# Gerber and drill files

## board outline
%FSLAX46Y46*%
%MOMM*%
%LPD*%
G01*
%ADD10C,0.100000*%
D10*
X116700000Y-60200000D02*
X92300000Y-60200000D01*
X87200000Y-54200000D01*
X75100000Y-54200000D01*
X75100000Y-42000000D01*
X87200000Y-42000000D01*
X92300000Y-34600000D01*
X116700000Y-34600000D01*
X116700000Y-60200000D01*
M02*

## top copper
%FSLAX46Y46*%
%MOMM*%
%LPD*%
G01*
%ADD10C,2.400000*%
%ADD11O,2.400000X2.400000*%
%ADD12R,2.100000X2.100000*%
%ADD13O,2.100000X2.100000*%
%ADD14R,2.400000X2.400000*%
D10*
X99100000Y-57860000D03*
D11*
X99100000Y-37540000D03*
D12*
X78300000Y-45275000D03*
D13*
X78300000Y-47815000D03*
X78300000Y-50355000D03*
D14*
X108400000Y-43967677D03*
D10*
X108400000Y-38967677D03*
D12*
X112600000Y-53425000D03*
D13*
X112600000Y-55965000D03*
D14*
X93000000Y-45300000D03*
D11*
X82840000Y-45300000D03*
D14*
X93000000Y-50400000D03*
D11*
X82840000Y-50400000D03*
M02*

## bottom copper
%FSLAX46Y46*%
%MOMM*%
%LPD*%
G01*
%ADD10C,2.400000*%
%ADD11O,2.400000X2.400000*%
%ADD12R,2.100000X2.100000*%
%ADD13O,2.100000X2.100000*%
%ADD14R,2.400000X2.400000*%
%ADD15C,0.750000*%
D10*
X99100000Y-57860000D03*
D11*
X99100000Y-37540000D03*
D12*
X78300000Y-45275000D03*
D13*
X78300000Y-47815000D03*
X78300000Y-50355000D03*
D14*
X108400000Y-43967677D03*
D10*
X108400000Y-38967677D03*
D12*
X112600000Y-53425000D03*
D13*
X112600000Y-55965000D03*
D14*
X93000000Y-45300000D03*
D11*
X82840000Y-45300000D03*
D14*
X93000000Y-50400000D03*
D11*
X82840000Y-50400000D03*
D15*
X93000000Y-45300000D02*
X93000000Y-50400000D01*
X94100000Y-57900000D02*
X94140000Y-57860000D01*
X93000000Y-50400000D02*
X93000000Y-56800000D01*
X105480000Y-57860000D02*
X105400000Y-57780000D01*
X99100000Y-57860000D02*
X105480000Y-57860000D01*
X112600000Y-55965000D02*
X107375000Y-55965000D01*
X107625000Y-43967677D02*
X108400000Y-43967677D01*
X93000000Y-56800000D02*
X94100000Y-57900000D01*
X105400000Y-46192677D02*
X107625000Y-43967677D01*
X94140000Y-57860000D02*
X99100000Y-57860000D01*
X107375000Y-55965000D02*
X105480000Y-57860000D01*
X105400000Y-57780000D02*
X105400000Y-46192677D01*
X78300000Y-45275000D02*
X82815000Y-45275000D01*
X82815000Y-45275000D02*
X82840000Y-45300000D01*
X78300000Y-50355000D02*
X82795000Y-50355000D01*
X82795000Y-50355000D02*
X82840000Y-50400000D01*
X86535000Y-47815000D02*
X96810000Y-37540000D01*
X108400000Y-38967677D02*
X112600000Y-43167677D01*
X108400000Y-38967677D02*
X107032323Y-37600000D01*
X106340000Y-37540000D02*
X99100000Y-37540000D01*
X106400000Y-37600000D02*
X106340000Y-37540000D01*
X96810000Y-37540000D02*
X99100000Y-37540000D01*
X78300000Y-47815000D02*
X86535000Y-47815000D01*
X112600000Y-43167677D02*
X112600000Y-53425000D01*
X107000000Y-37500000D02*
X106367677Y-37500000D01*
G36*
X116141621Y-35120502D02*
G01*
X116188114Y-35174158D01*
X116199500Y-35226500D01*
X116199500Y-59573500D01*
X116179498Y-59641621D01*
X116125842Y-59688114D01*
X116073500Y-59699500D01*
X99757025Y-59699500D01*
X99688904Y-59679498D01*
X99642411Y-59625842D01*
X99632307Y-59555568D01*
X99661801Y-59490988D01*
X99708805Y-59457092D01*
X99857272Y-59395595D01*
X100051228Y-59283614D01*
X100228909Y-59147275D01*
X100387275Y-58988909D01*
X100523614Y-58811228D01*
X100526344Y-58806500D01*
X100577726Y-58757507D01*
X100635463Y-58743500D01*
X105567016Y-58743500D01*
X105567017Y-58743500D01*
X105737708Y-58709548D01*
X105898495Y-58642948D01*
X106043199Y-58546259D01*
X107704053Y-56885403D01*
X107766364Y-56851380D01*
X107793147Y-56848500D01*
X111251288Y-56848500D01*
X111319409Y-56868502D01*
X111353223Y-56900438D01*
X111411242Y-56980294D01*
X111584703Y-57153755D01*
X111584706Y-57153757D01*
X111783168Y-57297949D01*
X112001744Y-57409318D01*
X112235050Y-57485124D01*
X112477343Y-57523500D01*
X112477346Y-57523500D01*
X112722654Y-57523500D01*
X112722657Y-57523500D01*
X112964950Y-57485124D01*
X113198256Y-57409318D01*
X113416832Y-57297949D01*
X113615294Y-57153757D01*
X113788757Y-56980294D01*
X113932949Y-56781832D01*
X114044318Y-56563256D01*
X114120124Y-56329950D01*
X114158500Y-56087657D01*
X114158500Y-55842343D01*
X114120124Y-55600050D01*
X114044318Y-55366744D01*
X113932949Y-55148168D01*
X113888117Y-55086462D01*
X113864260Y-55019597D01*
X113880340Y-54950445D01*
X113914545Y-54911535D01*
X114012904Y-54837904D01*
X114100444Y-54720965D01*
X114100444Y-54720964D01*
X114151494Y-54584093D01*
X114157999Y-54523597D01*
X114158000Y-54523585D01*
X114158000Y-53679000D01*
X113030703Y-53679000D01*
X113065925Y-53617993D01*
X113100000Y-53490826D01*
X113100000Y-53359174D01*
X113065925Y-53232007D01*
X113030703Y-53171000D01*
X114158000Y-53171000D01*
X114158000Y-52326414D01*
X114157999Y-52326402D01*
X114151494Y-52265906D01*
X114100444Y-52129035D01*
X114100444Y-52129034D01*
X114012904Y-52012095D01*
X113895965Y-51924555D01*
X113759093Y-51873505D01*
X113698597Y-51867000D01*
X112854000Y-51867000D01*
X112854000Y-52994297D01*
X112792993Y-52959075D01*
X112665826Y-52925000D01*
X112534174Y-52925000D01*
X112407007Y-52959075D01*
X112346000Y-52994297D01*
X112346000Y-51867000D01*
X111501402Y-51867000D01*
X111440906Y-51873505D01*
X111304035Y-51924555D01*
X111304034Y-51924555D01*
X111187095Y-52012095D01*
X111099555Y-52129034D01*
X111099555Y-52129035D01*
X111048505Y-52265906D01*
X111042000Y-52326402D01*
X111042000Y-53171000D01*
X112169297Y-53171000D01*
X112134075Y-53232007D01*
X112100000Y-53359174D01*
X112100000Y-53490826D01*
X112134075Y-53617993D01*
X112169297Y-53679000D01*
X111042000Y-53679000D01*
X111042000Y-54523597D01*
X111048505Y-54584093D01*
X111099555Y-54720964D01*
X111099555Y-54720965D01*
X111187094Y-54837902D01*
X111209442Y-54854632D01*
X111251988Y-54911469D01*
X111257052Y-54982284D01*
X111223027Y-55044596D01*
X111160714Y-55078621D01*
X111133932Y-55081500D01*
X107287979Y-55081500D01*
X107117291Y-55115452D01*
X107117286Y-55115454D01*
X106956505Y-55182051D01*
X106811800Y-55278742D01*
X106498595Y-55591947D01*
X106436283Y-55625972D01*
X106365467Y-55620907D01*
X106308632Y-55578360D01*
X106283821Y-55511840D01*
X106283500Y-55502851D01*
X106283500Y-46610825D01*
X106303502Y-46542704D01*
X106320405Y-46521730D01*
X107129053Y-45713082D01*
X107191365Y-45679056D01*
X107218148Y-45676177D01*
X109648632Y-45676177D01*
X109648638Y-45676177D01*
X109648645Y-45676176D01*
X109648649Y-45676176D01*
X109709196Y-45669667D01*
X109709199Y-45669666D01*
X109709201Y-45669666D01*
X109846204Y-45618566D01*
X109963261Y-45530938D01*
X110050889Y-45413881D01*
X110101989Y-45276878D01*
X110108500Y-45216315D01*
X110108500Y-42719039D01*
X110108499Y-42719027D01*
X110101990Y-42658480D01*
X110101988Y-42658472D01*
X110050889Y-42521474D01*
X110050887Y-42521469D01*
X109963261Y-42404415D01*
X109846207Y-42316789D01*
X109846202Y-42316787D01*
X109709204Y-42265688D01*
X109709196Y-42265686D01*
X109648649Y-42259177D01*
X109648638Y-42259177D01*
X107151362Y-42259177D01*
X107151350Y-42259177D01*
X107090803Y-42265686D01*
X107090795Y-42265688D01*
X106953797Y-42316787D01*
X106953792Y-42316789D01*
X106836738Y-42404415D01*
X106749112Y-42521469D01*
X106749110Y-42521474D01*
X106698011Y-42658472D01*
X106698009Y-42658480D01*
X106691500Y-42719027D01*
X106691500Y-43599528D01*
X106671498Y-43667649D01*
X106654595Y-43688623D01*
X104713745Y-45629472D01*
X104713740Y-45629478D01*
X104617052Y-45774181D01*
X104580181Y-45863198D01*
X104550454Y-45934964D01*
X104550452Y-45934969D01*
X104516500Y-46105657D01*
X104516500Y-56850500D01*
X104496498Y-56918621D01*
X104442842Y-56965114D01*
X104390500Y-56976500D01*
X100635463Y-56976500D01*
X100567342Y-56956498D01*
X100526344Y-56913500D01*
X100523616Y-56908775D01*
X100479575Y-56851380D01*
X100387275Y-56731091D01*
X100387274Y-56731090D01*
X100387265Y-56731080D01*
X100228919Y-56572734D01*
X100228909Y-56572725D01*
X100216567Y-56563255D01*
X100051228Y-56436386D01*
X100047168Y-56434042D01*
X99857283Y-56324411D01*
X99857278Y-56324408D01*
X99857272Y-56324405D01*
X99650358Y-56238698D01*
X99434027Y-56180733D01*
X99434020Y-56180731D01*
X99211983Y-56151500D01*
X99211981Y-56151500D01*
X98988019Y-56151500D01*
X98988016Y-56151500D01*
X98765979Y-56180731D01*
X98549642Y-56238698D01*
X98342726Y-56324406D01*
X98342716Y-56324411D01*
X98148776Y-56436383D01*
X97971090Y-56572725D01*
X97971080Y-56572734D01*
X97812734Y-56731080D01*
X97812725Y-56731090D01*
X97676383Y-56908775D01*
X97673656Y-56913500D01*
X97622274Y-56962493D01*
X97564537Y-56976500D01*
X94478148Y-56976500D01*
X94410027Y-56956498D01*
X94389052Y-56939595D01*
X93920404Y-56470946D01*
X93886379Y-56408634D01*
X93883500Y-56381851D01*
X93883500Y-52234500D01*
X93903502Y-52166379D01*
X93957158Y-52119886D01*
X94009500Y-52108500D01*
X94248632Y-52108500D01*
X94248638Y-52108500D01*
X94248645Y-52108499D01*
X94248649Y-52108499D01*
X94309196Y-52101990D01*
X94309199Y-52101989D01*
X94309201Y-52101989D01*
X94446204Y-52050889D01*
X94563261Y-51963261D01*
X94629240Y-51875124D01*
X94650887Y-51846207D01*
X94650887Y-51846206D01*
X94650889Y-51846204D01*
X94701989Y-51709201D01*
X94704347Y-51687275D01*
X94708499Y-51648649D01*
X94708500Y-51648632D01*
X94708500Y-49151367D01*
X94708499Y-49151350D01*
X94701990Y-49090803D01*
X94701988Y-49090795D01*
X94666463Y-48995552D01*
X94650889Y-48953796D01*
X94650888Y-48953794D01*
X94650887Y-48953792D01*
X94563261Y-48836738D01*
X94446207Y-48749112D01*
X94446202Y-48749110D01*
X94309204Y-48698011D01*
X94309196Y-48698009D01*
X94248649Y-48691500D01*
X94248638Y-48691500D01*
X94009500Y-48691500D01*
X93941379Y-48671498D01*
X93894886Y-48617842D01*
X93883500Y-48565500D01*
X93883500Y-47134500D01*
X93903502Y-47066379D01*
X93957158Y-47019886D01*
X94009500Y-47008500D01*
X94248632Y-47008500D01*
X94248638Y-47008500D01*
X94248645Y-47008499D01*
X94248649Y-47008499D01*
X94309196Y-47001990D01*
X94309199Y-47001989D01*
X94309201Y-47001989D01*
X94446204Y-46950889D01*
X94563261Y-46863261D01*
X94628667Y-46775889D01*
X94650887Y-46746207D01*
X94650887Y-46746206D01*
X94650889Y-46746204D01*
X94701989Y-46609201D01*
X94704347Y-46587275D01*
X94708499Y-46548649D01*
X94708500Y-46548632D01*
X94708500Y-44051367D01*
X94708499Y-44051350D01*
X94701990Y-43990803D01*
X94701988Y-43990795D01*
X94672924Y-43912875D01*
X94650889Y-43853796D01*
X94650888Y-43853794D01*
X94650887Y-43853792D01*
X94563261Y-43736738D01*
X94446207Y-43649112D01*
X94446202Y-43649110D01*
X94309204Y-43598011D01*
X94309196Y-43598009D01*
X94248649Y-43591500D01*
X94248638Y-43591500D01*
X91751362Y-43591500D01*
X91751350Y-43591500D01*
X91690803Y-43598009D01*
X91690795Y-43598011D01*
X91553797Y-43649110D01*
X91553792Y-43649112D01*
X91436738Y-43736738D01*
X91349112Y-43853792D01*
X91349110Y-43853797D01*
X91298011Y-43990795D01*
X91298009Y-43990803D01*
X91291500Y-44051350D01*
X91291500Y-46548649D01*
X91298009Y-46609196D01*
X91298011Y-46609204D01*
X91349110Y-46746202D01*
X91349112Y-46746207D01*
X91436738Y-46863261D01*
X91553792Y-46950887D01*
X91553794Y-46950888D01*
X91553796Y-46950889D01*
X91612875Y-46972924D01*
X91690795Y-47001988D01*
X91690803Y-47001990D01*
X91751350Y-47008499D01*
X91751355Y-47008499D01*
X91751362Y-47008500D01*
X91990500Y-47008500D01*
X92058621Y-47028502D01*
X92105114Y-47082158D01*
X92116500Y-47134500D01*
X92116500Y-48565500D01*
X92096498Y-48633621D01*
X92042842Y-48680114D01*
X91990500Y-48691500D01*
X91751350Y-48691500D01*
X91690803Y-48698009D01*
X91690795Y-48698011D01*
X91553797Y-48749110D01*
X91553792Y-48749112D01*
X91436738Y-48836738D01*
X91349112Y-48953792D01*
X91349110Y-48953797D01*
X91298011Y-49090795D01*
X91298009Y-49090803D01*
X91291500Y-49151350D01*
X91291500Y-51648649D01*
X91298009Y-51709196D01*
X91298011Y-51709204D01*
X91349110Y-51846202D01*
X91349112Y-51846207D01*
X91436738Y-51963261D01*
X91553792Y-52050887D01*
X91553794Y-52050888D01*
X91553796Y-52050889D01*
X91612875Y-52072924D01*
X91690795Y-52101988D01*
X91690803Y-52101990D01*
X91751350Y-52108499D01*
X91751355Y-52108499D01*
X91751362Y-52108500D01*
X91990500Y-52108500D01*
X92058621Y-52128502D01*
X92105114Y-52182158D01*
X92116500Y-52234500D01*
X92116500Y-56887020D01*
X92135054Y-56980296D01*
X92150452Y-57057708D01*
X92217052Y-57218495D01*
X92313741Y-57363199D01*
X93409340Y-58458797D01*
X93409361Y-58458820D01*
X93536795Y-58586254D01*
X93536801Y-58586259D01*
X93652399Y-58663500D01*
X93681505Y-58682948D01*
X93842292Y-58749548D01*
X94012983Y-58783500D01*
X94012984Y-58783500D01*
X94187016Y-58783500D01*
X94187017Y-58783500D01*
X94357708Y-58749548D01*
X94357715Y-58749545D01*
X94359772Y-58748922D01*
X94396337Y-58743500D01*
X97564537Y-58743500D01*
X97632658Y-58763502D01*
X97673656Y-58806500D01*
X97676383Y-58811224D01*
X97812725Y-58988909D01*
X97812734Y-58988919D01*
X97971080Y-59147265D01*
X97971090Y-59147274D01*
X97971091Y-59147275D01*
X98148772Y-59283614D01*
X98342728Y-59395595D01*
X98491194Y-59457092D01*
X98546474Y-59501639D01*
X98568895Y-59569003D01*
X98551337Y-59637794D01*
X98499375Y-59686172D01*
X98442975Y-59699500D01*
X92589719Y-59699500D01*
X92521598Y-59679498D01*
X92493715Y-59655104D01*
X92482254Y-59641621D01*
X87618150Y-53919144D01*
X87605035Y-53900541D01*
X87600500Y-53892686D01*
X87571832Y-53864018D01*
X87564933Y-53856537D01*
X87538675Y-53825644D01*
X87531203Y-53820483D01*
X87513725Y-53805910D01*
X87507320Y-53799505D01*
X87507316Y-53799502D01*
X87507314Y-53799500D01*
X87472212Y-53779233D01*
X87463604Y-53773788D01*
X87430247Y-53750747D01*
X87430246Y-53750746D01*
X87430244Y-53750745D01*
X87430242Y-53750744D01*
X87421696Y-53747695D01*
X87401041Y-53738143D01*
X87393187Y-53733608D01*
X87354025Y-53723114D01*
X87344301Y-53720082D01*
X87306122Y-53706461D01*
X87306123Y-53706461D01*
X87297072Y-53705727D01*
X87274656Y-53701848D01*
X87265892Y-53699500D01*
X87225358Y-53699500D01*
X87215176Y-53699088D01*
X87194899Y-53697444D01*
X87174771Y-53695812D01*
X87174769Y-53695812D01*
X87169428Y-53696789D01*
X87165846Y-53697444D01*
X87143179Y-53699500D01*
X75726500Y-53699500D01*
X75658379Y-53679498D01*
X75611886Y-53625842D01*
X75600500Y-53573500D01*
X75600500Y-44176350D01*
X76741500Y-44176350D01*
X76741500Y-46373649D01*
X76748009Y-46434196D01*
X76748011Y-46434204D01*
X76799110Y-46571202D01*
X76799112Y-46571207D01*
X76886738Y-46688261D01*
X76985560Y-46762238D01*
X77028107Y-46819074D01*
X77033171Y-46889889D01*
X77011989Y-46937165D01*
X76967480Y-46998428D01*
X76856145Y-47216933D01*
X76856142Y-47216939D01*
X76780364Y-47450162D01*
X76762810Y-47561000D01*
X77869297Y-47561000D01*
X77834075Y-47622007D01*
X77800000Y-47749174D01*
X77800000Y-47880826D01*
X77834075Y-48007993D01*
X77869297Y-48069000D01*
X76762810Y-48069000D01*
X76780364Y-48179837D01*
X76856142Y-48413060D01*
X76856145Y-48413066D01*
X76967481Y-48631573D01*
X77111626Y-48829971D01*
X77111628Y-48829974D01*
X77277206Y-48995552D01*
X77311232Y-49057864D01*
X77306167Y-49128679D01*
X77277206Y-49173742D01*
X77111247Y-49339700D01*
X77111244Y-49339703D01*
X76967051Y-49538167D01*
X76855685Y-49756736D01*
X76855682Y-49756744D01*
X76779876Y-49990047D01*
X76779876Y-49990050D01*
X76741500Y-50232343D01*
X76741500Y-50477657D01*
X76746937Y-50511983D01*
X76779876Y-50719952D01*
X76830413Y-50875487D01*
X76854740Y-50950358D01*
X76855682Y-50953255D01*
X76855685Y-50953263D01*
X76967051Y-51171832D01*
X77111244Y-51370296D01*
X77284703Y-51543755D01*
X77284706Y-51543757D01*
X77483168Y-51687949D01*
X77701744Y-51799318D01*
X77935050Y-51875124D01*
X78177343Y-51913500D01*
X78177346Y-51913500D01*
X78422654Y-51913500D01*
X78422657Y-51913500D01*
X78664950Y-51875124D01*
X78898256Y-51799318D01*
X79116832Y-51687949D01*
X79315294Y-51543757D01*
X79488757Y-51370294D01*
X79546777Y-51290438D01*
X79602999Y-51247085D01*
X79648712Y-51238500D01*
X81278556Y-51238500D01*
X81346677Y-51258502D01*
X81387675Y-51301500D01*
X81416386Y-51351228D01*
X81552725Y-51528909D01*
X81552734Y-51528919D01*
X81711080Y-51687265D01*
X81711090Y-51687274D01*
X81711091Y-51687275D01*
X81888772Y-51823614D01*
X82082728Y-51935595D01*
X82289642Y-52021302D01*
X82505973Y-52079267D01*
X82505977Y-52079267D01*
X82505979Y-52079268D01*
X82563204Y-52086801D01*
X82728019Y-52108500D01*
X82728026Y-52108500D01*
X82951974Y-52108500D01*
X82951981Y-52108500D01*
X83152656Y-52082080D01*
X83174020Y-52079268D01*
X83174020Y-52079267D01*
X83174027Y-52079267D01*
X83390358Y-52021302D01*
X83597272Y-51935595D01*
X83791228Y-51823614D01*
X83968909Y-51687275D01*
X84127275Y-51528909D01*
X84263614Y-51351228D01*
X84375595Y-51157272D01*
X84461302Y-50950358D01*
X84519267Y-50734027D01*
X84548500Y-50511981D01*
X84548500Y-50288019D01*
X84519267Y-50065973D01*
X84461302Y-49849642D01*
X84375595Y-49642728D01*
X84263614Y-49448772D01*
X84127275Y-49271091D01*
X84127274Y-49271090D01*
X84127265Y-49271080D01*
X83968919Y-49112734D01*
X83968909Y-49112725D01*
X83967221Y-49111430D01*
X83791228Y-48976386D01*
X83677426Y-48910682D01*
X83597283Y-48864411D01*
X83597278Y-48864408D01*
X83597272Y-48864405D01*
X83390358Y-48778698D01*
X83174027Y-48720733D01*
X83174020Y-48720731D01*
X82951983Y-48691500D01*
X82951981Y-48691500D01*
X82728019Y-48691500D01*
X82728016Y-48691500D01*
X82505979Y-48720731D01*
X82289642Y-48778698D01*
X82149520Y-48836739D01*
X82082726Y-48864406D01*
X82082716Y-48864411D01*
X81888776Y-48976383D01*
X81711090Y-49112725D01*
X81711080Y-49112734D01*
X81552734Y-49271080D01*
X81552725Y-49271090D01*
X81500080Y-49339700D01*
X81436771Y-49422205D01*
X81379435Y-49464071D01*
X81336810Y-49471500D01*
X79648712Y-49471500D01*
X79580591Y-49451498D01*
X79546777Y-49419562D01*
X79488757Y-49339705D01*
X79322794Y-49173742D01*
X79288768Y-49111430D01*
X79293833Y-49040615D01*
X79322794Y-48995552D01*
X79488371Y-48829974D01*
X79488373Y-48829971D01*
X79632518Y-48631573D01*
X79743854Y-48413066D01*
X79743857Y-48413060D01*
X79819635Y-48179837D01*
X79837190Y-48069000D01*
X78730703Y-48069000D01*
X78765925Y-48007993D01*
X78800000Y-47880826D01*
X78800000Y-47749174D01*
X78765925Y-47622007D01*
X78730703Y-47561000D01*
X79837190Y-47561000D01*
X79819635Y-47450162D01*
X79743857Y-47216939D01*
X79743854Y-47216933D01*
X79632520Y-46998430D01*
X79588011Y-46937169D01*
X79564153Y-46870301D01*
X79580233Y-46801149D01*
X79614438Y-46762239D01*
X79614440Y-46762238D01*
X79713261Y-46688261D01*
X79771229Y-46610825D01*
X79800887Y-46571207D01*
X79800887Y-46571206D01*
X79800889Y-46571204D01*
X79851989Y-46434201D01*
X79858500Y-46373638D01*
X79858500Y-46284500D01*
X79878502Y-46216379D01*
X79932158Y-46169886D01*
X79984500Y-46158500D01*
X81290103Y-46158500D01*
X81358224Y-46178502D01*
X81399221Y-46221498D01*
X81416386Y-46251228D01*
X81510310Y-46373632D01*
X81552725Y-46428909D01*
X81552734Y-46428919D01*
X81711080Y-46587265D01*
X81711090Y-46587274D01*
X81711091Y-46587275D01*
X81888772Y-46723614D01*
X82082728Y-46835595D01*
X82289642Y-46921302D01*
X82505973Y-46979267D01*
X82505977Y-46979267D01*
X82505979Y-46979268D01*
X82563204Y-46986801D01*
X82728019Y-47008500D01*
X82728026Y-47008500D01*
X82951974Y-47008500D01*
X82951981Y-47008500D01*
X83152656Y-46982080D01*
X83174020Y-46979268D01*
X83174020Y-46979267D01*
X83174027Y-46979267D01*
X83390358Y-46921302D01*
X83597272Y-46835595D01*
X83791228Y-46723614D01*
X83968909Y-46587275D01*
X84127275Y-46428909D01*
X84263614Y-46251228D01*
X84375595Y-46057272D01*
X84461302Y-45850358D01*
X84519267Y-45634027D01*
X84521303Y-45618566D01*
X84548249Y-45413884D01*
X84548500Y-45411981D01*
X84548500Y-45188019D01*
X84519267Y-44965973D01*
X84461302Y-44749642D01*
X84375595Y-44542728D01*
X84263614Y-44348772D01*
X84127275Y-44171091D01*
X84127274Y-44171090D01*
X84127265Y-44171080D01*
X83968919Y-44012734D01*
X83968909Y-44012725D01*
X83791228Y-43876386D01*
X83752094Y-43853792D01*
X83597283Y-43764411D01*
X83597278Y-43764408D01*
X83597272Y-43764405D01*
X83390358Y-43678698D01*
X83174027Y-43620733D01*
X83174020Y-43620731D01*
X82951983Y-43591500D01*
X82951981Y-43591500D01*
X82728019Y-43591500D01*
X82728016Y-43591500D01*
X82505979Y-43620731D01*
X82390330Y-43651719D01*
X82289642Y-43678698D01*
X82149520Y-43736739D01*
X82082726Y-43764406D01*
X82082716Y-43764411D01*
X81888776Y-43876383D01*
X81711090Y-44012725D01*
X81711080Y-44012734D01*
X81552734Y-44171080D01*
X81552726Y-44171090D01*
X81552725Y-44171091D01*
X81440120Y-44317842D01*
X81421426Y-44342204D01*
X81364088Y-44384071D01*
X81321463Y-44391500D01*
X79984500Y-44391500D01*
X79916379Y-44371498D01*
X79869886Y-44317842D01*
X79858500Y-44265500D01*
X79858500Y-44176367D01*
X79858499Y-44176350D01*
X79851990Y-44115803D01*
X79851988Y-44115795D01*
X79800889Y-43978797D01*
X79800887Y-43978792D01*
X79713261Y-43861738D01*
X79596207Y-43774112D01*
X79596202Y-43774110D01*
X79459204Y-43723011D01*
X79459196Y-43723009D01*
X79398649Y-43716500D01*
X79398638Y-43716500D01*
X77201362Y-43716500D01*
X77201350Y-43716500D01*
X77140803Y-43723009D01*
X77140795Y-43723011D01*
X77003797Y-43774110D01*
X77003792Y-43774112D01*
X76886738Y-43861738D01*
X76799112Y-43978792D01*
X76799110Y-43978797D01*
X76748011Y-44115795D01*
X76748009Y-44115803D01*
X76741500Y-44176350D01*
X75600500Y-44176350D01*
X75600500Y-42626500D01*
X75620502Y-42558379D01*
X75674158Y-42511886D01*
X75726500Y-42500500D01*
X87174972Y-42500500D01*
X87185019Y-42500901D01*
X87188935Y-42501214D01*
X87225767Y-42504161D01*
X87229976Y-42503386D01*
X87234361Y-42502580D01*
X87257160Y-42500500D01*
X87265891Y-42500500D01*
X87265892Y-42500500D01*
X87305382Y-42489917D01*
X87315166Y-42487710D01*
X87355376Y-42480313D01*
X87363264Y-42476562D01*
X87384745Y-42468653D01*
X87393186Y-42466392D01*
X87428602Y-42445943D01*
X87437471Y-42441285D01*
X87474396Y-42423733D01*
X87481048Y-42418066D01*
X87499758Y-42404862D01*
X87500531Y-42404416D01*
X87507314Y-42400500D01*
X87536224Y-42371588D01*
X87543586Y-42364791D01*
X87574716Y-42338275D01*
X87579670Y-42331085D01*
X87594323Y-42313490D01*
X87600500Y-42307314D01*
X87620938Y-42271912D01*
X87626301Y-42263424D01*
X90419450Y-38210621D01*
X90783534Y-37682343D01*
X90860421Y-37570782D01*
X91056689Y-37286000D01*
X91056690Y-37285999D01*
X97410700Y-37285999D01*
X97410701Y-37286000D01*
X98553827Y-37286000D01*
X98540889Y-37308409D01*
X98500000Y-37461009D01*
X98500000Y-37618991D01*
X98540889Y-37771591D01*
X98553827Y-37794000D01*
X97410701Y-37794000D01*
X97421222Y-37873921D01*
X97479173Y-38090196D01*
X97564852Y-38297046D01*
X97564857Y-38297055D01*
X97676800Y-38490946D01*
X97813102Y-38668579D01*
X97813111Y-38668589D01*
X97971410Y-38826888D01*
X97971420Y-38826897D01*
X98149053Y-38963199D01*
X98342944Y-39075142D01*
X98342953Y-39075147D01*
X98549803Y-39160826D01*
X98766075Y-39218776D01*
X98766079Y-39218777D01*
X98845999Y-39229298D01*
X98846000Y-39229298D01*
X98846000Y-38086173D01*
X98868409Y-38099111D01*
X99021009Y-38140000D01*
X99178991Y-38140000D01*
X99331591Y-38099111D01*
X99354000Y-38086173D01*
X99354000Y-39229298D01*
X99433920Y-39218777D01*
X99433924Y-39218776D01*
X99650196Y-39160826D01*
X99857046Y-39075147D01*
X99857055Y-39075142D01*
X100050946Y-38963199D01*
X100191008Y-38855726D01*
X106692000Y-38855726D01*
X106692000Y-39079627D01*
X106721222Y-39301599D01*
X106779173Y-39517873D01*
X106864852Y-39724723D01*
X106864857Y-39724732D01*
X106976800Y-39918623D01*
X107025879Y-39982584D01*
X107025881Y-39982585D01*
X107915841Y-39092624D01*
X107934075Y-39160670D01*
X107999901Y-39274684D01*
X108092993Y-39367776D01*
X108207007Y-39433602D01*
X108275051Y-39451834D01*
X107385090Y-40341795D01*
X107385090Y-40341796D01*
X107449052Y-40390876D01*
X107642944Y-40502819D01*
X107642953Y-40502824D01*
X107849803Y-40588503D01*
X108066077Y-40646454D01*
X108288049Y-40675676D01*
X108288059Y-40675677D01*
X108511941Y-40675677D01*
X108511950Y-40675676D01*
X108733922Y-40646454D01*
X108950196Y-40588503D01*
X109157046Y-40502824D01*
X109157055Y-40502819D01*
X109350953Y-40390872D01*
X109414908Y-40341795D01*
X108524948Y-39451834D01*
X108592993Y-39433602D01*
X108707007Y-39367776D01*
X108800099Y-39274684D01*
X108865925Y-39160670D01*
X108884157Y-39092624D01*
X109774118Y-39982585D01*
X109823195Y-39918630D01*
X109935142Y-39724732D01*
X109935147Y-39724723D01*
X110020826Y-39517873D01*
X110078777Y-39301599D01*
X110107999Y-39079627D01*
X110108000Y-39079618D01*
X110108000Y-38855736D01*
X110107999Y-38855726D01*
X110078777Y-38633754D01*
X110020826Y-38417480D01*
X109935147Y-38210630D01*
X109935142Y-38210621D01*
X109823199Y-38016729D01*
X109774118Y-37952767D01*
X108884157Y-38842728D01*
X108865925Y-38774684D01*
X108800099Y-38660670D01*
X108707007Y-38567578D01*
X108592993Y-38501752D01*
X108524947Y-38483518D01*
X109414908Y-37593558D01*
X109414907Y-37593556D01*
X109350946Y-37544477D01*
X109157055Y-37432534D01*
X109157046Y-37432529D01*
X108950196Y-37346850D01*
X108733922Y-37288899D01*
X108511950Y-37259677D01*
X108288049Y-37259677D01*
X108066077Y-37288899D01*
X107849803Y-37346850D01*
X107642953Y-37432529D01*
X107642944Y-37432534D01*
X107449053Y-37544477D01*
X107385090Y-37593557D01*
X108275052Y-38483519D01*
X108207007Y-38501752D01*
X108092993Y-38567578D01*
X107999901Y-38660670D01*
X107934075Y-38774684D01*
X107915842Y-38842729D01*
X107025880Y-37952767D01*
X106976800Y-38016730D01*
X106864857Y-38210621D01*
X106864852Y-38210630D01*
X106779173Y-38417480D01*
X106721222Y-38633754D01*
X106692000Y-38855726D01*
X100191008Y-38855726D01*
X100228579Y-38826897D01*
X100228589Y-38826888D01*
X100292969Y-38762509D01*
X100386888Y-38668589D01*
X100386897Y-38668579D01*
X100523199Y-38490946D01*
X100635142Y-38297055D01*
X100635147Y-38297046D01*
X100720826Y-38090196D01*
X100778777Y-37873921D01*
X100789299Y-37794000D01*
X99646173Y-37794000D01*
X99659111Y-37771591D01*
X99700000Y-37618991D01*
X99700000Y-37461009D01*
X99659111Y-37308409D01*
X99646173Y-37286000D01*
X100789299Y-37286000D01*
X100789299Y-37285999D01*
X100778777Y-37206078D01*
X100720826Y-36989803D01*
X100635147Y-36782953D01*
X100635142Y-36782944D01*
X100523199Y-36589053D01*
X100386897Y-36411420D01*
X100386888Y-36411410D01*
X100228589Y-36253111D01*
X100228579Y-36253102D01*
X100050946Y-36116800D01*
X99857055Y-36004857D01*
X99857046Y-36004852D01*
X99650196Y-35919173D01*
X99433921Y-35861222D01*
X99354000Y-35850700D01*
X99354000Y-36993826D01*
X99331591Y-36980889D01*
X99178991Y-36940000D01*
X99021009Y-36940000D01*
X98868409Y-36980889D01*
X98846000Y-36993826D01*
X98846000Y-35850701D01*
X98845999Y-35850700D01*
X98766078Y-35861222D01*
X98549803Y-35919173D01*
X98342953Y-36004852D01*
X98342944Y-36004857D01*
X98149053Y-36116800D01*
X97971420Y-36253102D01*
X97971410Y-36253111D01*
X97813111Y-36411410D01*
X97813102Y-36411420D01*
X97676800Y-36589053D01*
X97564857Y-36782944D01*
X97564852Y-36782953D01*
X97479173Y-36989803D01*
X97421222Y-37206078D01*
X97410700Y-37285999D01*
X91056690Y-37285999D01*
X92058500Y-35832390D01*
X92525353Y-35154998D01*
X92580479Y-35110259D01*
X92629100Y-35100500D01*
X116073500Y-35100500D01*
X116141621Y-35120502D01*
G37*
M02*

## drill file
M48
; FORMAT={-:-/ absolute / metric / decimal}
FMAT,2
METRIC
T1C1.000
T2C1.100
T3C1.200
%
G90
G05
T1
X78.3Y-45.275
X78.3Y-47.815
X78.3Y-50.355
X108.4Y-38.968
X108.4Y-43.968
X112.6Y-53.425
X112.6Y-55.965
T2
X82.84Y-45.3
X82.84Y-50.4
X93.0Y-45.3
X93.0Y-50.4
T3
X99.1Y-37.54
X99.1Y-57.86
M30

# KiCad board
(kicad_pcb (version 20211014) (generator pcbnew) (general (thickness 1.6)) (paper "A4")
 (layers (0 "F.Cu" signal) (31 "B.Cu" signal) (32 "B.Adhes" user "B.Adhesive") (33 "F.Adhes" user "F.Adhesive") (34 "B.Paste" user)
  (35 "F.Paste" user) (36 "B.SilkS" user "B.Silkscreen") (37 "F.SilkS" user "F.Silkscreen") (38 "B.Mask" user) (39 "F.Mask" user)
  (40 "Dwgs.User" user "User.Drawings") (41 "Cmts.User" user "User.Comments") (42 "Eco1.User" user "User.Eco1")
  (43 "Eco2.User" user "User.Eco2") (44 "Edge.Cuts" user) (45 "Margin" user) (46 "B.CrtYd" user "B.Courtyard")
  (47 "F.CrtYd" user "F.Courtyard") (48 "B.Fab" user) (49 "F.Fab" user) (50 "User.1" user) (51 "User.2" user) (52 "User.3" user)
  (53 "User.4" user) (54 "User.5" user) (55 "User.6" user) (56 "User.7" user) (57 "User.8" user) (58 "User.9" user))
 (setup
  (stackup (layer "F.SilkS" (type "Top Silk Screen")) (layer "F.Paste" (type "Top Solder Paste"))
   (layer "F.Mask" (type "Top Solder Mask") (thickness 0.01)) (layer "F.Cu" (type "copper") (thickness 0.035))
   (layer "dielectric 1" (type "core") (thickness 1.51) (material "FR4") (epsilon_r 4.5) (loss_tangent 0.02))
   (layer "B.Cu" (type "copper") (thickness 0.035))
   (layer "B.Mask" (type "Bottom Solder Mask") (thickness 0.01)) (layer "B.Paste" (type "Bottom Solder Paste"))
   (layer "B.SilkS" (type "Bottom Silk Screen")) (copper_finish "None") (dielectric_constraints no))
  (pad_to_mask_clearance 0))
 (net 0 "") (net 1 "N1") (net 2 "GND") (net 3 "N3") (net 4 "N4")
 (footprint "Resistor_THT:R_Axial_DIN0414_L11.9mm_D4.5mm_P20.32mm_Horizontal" (layer "F.Cu") (at 99.1 57.86 90)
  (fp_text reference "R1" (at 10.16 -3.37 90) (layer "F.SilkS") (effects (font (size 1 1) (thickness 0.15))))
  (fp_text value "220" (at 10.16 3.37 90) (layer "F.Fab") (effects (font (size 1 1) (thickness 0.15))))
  (pad "1" thru_hole circle (at 0 0 90) (size 2.4 2.4) (drill 1.2) (layers *.Cu *.Mask) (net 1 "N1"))
  (pad "2" thru_hole oval (at 20.32 0 90) (size 2.4 2.4) (drill 1.2) (layers *.Cu *.Mask) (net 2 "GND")))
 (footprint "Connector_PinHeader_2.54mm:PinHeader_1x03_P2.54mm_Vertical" (layer "F.Cu") (at 78.3 45.275)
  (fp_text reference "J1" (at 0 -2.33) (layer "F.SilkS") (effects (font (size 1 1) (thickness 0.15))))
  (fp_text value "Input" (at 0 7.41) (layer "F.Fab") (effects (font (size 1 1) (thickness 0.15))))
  (pad "1" thru_hole rect (at 0 0) (size 2.1 2.1) (drill 1) (layers *.Cu *.Mask) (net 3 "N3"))
  (pad "2" thru_hole oval (at 0 2.54) (size 2.1 2.1) (drill 1) (layers *.Cu *.Mask) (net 2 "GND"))
  (pad "3" thru_hole oval (at 0 5.08) (size 2.1 2.1) (drill 1) (layers *.Cu *.Mask) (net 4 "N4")))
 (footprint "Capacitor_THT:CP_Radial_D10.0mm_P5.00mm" (layer "F.Cu") (at 108.4 43.967677 90)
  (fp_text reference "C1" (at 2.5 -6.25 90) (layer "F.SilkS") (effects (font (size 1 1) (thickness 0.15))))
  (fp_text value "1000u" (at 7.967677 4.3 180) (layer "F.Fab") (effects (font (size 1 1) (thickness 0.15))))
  (pad "1" thru_hole rect (at 0 0 90) (size 2.4 2.4) (drill 1) (layers *.Cu *.Mask) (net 1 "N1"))
  (pad "2" thru_hole circle (at 5 0 90) (size 2.4 2.4) (drill 1) (layers *.Cu *.Mask) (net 2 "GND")))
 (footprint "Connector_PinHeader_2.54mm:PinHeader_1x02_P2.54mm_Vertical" (layer "F.Cu") (at 112.6 53.425)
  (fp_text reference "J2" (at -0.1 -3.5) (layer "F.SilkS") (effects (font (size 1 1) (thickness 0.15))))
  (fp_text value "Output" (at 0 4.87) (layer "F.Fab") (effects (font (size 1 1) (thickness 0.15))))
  (pad "1" thru_hole rect (at 0 0) (size 2.1 2.1) (drill 1) (layers *.Cu *.Mask) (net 2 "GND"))
  (pad "2" thru_hole oval (at 0 2.54) (size 2.1 2.1) (drill 1) (layers *.Cu *.Mask) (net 1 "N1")))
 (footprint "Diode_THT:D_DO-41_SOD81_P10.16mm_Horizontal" (layer "F.Cu") (at 93 45.3 180)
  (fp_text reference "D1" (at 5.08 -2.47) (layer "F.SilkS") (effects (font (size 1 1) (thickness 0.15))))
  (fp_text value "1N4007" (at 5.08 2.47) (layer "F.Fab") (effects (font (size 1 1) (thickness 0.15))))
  (pad "1" thru_hole rect (at 0 0 180) (size 2.4 2.4) (drill 1.1) (layers *.Cu *.Mask) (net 1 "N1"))
  (pad "2" thru_hole oval (at 10.16 0 180) (size 2.4 2.4) (drill 1.1) (layers *.Cu *.Mask) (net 3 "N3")))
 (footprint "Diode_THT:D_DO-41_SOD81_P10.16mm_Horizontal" (layer "F.Cu") (at 93 50.4 180)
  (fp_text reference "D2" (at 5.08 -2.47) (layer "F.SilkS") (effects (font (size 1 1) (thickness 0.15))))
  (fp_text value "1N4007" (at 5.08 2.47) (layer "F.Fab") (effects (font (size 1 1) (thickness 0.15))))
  (pad "1" thru_hole rect (at 0 0 180) (size 2.4 2.4) (drill 1.1) (layers *.Cu *.Mask) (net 1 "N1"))
  (pad "2" thru_hole oval (at 10.16 0 180) (size 2.4 2.4) (drill 1.1) (layers *.Cu *.Mask) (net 4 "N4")))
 (gr_poly
  (pts (xy 116.7 60.2) (xy 92.3 60.2) (xy 87.2 54.2) (xy 75.1 54.2) (xy 75.1 42) (xy 87.2 42) (xy 92.3 34.6) (xy 116.7 34.6))
  (layer "Edge.Cuts") (width 0.1) (fill none))
 (segment (start 93 45.3) (end 93 50.4) (width 0.75) (layer "B.Cu") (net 1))
 (segment (start 94.1 57.9) (end 94.14 57.86) (width 0.75) (layer "B.Cu") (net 1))
 (segment (start 93 50.4) (end 93 56.8) (width 0.75) (layer "B.Cu") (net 1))
 (segment (start 105.48 57.86) (end 105.4 57.78) (width 0.75) (layer "B.Cu") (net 1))
 (segment (start 99.1 57.86) (end 105.48 57.86) (width 0.75) (layer "B.Cu") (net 1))
 (segment (start 112.6 55.965) (end 107.375 55.965) (width 0.75) (layer "B.Cu") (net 1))
 (segment (start 107.625 43.967677) (end 108.4 43.967677) (width 0.75) (layer "B.Cu") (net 1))
 (segment (start 93 56.8) (end 94.1 57.9) (width 0.75) (layer "B.Cu") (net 1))
 (segment (start 105.4 46.192677) (end 107.625 43.967677) (width 0.75) (layer "B.Cu") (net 1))
 (segment (start 94.14 57.86) (end 99.1 57.86) (width 0.75) (layer "B.Cu") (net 1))
 (segment (start 107.375 55.965) (end 105.48 57.86) (width 0.75) (layer "B.Cu") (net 1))
 (segment (start 105.4 57.78) (end 105.4 46.192677) (width 0.75) (layer "B.Cu") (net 1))
 (segment (start 78.3 45.275) (end 82.815 45.275) (width 0.75) (layer "B.Cu") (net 3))
 (segment (start 82.815 45.275) (end 82.84 45.3) (width 0.75) (layer "B.Cu") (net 3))
 (segment (start 78.3 50.355) (end 82.795 50.355) (width 0.75) (layer "B.Cu") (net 4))
 (segment (start 82.795 50.355) (end 82.84 50.4) (width 0.75) (layer "B.Cu") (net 4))
 (segment (start 86.535 47.815) (end 96.81 37.54) (width 0.75) (layer "B.Cu") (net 2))
 (segment (start 108.4 38.967677) (end 112.6 43.167677) (width 0.75) (layer "B.Cu") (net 2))
 (segment (start 108.4 38.967677) (end 107.032323 37.6) (width 0.75) (layer "B.Cu") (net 2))
 (segment (start 106.34 37.54) (end 99.1 37.54) (width 0.75) (layer "B.Cu") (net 2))
 (segment (start 106.4 37.6) (end 106.34 37.54) (width 0.75) (layer "B.Cu") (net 2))
 (segment (start 96.81 37.54) (end 99.1 37.54) (width 0.75) (layer "B.Cu") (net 2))
 (segment (start 78.3 47.815) (end 86.535 47.815) (width 0.75) (layer "B.Cu") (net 2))
 (segment (start 112.6 43.167677) (end 112.6 53.425) (width 0.75) (layer "B.Cu") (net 2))
 (segment (start 107 37.5) (end 106.367677 37.5) (width 0.75) (layer "B.Cu") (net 2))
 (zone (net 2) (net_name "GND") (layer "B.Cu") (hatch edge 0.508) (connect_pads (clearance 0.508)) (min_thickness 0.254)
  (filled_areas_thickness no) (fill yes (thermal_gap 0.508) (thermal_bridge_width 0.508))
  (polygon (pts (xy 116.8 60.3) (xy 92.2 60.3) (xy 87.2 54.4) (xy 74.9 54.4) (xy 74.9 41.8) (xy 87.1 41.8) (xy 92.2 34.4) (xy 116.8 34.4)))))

